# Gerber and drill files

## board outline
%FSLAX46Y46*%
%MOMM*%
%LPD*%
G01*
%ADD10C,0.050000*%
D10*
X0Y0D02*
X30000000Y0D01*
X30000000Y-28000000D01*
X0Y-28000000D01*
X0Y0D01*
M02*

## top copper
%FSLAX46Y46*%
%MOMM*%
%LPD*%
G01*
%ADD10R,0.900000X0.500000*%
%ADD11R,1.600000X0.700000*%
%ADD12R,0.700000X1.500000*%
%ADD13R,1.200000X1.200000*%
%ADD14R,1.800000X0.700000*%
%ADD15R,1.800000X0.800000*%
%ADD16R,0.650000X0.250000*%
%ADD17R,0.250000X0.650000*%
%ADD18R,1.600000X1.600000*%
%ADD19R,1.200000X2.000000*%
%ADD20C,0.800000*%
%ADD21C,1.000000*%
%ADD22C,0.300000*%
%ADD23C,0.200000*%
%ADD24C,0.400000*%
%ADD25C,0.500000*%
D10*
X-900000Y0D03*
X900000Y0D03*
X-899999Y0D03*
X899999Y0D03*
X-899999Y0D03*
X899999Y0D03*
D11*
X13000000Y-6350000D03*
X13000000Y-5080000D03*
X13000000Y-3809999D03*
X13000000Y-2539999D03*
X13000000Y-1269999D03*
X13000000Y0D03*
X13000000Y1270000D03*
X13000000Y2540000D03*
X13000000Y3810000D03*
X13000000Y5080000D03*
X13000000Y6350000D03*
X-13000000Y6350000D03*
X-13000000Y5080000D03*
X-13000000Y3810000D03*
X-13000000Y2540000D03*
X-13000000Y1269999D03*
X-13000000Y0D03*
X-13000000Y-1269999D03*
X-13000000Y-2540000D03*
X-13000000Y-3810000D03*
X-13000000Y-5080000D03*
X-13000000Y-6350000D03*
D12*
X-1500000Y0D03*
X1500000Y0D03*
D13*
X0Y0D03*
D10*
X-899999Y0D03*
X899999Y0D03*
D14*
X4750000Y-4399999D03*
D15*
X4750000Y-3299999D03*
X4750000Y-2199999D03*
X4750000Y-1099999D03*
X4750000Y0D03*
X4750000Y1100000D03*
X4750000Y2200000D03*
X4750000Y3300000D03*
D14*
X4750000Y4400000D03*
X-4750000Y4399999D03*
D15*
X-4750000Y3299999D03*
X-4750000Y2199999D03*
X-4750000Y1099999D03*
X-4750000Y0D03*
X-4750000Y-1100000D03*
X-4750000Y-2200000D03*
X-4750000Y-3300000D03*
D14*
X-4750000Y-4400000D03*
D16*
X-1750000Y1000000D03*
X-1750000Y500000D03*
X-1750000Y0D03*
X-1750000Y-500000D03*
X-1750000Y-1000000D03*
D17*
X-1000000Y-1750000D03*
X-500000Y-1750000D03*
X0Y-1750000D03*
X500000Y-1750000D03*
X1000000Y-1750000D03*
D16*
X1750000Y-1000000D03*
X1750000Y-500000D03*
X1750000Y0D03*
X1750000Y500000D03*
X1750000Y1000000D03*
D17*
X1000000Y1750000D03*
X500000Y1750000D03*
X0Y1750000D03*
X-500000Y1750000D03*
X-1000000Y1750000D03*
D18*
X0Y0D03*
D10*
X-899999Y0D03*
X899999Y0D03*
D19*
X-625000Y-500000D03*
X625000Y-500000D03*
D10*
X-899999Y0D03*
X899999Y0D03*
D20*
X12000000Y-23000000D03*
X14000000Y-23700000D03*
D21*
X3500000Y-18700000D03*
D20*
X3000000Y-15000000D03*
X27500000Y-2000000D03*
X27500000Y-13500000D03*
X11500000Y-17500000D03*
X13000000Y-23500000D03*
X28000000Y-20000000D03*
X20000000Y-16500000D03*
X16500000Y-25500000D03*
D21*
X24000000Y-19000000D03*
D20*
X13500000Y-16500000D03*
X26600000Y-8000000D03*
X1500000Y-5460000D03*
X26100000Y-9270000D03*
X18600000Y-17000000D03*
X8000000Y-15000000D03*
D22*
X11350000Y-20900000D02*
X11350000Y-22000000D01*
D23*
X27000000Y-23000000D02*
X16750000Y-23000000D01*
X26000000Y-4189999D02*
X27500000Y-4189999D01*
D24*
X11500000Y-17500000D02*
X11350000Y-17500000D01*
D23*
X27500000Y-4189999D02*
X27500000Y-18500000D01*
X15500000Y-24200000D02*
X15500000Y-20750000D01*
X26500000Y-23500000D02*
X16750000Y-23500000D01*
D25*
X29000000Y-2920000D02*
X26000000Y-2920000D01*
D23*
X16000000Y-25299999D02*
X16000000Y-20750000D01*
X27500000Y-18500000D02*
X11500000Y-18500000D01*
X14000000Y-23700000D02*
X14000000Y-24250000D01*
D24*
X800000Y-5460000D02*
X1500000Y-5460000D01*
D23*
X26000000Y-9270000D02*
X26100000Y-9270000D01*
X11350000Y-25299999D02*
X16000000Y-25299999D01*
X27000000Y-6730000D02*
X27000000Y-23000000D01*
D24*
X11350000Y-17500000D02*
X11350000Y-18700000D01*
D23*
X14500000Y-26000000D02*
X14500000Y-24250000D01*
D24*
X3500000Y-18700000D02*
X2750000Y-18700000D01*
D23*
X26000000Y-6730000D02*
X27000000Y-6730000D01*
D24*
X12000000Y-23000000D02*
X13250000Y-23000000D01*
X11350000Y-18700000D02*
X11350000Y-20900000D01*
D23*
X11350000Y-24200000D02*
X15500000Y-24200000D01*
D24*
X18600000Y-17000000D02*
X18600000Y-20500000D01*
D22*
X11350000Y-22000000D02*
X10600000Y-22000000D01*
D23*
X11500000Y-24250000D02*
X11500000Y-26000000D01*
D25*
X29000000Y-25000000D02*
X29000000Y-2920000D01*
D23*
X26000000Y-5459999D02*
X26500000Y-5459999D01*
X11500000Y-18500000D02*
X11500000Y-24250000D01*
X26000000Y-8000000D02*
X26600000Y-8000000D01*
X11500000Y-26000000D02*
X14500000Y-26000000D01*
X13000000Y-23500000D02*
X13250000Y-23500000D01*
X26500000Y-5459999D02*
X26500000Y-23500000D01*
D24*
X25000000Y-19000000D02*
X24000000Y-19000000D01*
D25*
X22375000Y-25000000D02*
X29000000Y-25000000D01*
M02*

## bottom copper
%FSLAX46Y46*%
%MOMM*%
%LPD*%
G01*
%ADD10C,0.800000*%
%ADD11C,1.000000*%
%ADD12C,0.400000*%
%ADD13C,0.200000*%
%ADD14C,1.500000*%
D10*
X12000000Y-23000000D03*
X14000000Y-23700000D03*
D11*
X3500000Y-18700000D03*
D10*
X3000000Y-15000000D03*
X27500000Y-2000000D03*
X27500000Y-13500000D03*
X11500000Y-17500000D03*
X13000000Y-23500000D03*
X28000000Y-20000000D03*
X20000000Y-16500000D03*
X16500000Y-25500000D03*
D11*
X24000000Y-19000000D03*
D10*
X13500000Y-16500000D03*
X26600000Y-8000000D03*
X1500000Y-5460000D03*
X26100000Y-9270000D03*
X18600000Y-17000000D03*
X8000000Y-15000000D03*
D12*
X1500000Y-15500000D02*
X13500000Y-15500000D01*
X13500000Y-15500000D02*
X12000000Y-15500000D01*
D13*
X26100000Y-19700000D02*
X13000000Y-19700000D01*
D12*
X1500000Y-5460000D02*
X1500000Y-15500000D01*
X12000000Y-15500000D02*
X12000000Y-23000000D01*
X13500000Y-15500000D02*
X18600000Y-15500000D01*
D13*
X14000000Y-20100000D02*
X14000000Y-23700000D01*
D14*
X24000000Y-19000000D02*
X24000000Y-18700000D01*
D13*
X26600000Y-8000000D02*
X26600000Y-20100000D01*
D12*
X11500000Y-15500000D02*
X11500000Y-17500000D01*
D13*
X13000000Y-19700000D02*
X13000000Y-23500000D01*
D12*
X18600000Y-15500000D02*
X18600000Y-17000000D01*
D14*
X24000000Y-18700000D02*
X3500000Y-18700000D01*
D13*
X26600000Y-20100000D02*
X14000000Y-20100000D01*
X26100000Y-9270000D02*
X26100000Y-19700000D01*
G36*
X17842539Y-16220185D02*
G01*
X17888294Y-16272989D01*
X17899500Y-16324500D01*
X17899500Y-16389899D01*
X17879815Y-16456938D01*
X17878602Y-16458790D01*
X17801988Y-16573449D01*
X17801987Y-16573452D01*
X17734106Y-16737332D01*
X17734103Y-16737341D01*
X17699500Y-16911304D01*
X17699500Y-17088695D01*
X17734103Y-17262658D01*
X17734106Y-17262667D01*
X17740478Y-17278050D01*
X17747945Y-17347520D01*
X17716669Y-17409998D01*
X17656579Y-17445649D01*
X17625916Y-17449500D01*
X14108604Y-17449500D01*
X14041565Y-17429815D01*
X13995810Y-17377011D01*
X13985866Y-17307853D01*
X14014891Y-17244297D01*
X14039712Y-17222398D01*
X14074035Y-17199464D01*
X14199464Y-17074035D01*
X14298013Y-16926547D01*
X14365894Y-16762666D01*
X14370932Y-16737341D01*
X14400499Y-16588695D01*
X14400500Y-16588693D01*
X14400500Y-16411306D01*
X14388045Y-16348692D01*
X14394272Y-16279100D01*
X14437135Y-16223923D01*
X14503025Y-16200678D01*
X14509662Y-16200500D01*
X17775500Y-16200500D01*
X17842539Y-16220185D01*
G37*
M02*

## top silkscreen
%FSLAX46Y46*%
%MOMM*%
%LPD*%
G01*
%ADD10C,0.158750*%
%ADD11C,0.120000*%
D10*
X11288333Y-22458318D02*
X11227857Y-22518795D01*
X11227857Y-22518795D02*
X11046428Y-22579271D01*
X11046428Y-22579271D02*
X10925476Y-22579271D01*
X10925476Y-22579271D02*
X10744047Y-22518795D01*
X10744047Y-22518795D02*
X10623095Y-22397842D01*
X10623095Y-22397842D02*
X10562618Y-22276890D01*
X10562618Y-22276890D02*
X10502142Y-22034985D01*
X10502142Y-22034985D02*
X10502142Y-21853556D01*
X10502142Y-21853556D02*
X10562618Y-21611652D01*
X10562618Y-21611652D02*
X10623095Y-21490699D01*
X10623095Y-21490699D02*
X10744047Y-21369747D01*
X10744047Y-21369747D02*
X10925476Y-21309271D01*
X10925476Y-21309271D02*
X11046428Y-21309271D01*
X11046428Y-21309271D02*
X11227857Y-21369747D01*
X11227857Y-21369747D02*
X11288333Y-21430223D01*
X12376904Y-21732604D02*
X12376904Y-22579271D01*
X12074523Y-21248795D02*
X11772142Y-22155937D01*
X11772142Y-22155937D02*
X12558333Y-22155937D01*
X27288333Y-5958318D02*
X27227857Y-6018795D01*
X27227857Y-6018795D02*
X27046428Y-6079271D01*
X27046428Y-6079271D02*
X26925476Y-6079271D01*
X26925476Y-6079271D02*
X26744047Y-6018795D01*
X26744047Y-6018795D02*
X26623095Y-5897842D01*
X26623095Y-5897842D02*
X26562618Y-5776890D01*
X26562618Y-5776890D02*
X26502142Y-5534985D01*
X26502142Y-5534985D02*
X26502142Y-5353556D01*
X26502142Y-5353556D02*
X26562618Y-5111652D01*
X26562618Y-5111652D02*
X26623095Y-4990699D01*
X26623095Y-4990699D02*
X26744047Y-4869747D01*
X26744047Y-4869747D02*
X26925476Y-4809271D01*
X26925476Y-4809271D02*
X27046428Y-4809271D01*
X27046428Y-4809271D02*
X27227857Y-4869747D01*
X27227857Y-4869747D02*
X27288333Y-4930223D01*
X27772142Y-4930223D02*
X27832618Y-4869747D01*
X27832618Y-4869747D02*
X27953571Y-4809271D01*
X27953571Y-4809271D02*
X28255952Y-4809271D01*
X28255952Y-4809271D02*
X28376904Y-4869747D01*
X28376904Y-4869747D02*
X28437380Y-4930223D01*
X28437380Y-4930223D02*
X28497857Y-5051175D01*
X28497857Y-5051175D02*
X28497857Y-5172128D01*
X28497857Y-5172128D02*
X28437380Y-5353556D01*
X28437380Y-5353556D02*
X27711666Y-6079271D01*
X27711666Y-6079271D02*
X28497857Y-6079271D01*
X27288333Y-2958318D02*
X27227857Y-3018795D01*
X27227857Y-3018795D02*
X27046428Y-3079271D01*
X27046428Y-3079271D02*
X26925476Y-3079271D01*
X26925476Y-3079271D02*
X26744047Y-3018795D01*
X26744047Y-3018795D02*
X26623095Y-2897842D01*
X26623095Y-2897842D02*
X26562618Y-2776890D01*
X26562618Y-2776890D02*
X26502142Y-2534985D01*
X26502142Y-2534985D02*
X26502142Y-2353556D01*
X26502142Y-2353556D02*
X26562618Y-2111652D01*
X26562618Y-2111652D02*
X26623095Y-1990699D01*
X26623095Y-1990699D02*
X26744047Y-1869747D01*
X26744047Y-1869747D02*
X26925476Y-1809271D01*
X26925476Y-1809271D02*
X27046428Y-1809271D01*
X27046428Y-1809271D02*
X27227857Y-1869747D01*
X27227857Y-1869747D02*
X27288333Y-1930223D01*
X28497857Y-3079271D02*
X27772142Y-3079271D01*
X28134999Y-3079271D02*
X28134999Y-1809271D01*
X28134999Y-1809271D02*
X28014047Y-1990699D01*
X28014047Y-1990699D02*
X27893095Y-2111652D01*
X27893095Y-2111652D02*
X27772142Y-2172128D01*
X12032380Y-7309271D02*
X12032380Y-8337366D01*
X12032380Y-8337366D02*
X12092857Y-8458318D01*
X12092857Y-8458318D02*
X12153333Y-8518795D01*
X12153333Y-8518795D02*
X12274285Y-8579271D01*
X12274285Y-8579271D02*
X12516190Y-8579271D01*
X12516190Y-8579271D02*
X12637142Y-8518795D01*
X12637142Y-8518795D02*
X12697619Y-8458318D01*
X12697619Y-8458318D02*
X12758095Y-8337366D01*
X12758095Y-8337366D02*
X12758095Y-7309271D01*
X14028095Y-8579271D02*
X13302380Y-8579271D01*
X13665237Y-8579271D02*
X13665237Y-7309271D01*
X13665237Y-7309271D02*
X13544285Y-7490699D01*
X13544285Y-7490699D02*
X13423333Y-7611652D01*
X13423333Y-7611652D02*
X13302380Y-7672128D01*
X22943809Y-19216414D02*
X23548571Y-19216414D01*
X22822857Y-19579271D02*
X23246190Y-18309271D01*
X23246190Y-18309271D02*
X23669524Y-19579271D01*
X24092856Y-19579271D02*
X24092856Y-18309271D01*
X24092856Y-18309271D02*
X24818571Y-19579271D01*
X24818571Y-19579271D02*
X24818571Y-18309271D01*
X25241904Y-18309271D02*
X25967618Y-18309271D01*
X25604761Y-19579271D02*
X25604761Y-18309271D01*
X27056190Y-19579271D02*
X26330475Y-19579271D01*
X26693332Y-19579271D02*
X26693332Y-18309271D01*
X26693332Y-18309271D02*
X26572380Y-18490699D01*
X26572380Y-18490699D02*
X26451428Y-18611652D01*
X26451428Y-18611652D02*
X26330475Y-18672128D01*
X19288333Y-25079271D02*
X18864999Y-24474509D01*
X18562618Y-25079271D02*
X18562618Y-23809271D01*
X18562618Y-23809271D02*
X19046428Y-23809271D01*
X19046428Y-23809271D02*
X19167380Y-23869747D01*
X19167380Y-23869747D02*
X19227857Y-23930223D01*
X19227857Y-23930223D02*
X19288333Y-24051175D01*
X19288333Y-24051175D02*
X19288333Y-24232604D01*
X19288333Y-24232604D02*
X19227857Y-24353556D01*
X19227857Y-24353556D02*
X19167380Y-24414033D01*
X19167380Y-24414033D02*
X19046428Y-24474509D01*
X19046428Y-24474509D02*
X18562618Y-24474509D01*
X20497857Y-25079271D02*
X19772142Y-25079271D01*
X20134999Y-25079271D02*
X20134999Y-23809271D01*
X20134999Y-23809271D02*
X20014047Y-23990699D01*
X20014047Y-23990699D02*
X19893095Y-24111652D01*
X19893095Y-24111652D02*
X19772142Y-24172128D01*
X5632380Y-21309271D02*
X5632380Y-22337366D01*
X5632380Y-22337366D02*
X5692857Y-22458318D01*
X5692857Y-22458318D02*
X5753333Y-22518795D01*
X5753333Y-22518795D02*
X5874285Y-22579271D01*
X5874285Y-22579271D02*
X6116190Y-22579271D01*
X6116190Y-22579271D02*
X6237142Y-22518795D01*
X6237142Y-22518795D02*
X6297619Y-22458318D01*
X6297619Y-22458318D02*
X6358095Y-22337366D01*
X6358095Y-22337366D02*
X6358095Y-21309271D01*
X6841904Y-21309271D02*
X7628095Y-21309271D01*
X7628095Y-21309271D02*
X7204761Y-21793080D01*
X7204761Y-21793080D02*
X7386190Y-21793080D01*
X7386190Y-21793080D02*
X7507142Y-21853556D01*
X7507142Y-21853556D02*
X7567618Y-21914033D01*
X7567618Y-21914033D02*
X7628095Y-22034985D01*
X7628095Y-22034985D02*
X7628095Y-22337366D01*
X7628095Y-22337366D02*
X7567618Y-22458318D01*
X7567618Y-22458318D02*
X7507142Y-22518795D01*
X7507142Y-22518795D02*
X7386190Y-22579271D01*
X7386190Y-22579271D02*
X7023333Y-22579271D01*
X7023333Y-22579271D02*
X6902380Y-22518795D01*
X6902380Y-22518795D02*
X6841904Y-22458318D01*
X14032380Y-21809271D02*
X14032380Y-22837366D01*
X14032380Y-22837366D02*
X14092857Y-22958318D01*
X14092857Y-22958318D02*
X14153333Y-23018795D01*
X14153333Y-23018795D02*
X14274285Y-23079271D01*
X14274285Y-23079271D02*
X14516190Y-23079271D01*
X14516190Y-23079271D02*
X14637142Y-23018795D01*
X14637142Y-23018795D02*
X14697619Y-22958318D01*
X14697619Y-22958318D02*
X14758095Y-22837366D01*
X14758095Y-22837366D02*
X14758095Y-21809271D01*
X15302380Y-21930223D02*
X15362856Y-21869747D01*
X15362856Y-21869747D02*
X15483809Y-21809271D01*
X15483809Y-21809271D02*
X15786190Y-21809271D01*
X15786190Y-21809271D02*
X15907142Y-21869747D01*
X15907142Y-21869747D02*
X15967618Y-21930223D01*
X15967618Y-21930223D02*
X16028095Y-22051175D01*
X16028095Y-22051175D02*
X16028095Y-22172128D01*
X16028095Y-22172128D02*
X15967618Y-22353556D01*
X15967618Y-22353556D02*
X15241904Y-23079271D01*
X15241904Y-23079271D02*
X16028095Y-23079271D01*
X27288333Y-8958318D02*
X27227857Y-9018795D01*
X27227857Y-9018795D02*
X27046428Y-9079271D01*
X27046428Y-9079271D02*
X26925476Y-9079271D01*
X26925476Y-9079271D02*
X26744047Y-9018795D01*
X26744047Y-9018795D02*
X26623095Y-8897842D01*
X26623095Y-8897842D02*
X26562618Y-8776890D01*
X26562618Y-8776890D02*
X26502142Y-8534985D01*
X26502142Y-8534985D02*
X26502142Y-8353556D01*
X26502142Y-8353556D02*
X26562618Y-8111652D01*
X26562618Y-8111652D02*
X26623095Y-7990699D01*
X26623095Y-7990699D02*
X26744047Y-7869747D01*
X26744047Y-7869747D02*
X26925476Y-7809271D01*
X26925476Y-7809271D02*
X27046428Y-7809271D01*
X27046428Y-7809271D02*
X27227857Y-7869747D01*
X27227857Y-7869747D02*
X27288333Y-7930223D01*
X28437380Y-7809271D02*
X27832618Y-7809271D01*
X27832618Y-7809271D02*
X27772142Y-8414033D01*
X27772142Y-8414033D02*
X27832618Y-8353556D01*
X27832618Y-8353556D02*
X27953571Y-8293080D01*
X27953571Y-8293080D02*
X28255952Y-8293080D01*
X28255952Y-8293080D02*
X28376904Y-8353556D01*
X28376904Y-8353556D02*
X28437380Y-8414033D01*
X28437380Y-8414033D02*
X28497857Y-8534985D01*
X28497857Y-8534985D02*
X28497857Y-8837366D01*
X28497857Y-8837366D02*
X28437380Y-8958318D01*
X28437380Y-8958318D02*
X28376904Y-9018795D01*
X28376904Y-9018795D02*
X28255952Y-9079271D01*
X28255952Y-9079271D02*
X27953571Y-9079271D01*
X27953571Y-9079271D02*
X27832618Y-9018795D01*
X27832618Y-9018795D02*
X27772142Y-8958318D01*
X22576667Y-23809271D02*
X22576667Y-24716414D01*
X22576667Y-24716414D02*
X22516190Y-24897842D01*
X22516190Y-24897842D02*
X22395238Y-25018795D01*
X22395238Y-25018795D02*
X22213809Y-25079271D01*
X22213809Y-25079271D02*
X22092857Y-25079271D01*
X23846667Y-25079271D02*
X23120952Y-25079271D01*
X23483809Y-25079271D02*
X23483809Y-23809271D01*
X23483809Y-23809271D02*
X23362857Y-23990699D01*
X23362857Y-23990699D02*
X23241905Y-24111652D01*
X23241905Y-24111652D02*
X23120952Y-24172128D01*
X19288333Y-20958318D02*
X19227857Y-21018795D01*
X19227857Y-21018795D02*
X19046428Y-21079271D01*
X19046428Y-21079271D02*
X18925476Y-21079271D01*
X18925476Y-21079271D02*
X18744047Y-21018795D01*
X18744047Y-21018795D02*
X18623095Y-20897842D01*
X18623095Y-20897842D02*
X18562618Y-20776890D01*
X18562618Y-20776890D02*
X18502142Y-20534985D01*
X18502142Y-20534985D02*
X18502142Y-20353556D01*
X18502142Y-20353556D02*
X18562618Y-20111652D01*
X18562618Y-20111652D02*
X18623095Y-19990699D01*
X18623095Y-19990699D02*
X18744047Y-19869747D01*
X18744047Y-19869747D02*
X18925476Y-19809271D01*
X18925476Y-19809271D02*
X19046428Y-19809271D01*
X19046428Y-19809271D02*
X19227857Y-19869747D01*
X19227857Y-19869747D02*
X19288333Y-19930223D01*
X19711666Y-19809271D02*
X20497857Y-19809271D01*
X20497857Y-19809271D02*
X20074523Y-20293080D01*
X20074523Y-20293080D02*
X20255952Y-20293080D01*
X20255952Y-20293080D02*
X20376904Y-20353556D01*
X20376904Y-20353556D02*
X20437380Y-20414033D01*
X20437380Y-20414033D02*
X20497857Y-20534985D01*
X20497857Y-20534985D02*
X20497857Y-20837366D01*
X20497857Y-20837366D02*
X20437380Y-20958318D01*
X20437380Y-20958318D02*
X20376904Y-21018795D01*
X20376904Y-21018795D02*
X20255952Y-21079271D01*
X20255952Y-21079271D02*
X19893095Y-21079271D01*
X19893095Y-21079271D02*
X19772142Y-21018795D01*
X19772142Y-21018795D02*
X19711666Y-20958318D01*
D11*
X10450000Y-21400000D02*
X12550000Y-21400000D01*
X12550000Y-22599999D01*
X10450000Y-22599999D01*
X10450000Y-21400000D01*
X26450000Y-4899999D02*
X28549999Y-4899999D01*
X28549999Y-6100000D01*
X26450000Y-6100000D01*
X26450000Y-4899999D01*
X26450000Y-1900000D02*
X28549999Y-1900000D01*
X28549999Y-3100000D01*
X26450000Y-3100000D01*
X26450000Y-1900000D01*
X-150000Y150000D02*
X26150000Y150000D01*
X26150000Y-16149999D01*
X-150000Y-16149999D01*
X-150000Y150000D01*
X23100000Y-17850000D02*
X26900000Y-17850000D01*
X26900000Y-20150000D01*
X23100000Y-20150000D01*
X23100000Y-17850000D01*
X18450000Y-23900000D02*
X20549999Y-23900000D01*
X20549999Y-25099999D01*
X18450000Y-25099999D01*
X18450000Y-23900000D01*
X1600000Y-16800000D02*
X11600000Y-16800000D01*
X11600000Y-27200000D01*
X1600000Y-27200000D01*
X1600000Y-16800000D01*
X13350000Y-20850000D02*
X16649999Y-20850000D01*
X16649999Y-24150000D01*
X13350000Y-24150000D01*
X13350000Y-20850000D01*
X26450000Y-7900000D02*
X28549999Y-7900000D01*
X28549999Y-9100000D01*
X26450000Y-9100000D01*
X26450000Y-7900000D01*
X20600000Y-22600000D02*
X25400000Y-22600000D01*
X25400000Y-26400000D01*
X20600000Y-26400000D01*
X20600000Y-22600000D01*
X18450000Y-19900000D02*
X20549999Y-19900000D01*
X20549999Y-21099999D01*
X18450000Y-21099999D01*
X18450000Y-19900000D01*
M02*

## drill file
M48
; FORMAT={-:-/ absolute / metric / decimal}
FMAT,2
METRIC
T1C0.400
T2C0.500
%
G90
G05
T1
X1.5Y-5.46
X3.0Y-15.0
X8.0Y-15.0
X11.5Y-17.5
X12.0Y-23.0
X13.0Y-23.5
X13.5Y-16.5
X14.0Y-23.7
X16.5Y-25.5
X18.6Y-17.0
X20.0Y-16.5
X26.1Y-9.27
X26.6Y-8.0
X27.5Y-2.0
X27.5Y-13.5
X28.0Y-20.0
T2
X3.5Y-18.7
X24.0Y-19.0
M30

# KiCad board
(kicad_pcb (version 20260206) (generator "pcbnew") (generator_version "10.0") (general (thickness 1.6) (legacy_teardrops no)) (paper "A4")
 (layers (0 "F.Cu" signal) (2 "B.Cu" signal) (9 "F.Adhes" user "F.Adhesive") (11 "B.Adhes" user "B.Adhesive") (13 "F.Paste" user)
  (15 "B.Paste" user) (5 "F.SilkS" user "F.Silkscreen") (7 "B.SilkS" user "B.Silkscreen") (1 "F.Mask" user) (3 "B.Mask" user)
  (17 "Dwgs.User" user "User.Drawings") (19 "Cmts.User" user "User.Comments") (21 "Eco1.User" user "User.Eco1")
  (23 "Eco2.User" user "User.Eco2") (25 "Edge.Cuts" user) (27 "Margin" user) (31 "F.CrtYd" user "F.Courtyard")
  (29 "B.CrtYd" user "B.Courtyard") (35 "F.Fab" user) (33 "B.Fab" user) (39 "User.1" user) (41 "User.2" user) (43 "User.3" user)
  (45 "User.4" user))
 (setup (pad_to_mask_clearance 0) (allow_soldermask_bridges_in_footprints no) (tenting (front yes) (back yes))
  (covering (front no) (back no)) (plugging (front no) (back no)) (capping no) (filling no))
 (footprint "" (layer "F.Cu") (at 11.5 22)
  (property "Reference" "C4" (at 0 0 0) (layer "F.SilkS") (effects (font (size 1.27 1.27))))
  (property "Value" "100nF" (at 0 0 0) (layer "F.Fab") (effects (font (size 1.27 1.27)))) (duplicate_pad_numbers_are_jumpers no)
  (fp_rect (start -1.05 -0.6) (end 1.05 0.599999) (stroke (width 0.12) (type default)) (fill no) (layer "F.SilkS"))
  (pad "1" smd rect (at -12.4 -22) (size 0.9 0.5) (layers "F.Cu" "F.Mask" "F.Paste") (thermal_bridge_angle 45))
  (pad "2" smd rect (at -10.6 -22) (size 0.9 0.5) (layers "F.Cu" "F.Mask" "F.Paste") (thermal_bridge_angle 45)))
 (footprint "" (layer "F.Cu") (at 27.5 5.5)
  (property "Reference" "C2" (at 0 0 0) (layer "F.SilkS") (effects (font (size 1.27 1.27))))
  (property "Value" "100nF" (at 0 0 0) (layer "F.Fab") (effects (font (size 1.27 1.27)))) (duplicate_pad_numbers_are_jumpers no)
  (fp_rect (start -1.05 -0.600001) (end 1.049999 0.6) (stroke (width 0.12) (type default)) (fill no) (layer "F.SilkS"))
  (pad "1" smd rect (at -28.399999 -5.5) (size 0.9 0.5) (layers "F.Cu" "F.Mask" "F.Paste") (thermal_bridge_angle 45))
  (pad "2" smd rect (at -26.600001 -5.5) (size 0.9 0.5) (layers "F.Cu" "F.Mask" "F.Paste") (thermal_bridge_angle 45)))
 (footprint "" (layer "F.Cu") (at 27.5 2.5)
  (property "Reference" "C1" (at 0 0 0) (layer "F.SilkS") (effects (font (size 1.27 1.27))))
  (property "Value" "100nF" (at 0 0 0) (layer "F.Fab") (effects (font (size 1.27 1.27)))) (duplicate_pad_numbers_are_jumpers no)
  (fp_rect (start -1.05 -0.6) (end 1.049999 0.6) (stroke (width 0.12) (type default)) (fill no) (layer "F.SilkS"))
  (pad "1" smd rect (at -28.399999 -2.5) (size 0.9 0.5) (layers "F.Cu" "F.Mask" "F.Paste") (thermal_bridge_angle 45))
  (pad "2" smd rect (at -26.600001 -2.5) (size 0.9 0.5) (layers "F.Cu" "F.Mask" "F.Paste") (thermal_bridge_angle 45)))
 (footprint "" (layer "F.Cu") (at 13 8)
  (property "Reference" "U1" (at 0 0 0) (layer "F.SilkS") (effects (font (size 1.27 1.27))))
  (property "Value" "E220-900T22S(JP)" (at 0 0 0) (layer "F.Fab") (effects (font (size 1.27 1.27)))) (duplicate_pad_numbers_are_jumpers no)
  (fp_rect (start -13.15 -8.15) (end 13.15 8.149999) (stroke (width 0.12) (type default)) (fill no) (layer "F.SilkS"))
  (pad "1" smd rect (at 0 -1.65) (size 1.6 0.7) (layers "F.Cu" "F.Mask" "F.Paste") (thermal_bridge_angle 45))
  (pad "2" smd rect (at 0 -2.92) (size 1.6 0.7) (layers "F.Cu" "F.Mask" "F.Paste") (thermal_bridge_angle 45))
  (pad "3" smd rect (at 0 -4.190001) (size 1.6 0.7) (layers "F.Cu" "F.Mask" "F.Paste") (thermal_bridge_angle 45))
  (pad "4" smd rect (at 0 -5.460001) (size 1.6 0.7) (layers "F.Cu" "F.Mask" "F.Paste") (thermal_bridge_angle 45))
  (pad "5" smd rect (at 0 -6.730001) (size 1.6 0.7) (layers "F.Cu" "F.Mask" "F.Paste") (thermal_bridge_angle 45))
  (pad "6" smd rect (at 0 -8) (size 1.6 0.7) (layers "F.Cu" "F.Mask" "F.Paste") (thermal_bridge_angle 45))
  (pad "7" smd rect (at 0 -9.27) (size 1.6 0.7) (layers "F.Cu" "F.Mask" "F.Paste") (thermal_bridge_angle 45))
  (pad "8" smd rect (at 0 -10.54) (size 1.6 0.7) (layers "F.Cu" "F.Mask" "F.Paste") (thermal_bridge_angle 45))
  (pad "9" smd rect (at 0 -11.81) (size 1.6 0.7) (layers "F.Cu" "F.Mask" "F.Paste") (thermal_bridge_angle 45))
  (pad "10" smd rect (at 0 -13.08) (size 1.6 0.7) (layers "F.Cu" "F.Mask" "F.Paste") (thermal_bridge_angle 45))
  (pad "11" smd rect (at 0 -14.35) (size 1.6 0.7) (layers "F.Cu" "F.Mask" "F.Paste") (thermal_bridge_angle 45))
  (pad "12" smd rect (at -26 -14.35) (size 1.6 0.7) (layers "F.Cu" "F.Mask" "F.Paste") (thermal_bridge_angle 45))
  (pad "13" smd rect (at -26 -13.08) (size 1.6 0.7) (layers "F.Cu" "F.Mask" "F.Paste") (thermal_bridge_angle 45))
  (pad "14" smd rect (at -26 -11.81) (size 1.6 0.7) (layers "F.Cu" "F.Mask" "F.Paste") (thermal_bridge_angle 45))
  (pad "15" smd rect (at -26 -10.54) (size 1.6 0.7) (layers "F.Cu" "F.Mask" "F.Paste") (thermal_bridge_angle 45))
  (pad "16" smd rect (at -26 -9.269999) (size 1.6 0.7) (layers "F.Cu" "F.Mask" "F.Paste") (thermal_bridge_angle 45))
  (pad "17" smd rect (at -26 -8) (size 1.6 0.7) (layers "F.Cu" "F.Mask" "F.Paste") (thermal_bridge_angle 45))
  (pad "18" smd rect (at -26 -6.730001) (size 1.6 0.7) (layers "F.Cu" "F.Mask" "F.Paste") (thermal_bridge_angle 45))
  (pad "19" smd rect (at -26 -5.46) (size 1.6 0.7) (layers "F.Cu" "F.Mask" "F.Paste") (thermal_bridge_angle 45))
  (pad "20" smd rect (at -26 -4.19) (size 1.6 0.7) (layers "F.Cu" "F.Mask" "F.Paste") (thermal_bridge_angle 45))
  (pad "21" smd rect (at -26 -2.92) (size 1.6 0.7) (layers "F.Cu" "F.Mask" "F.Paste") (thermal_bridge_angle 45))
  (pad "22" smd rect (at -26 -1.65) (size 1.6 0.7) (layers "F.Cu" "F.Mask" "F.Paste") (thermal_bridge_angle 45)))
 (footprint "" (layer "F.Cu") (at 25 19)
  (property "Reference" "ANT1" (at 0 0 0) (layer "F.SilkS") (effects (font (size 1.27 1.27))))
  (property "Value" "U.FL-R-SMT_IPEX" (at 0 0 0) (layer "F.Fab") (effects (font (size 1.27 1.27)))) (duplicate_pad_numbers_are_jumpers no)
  (fp_rect (start -1.9 -1.15) (end 1.9 1.15) (stroke (width 0.12) (type default)) (fill no) (layer "F.SilkS"))
  (pad "G1" smd rect (at -26.5 -19) (size 0.7 1.5) (layers "F.Cu" "F.Mask" "F.Paste") (thermal_bridge_angle 45))
  (pad "G2" smd rect (at -23.5 -19) (size 0.7 1.5) (layers "F.Cu" "F.Mask" "F.Paste") (thermal_bridge_angle 45))
  (pad "S" smd rect (at -25 -19) (size 1.2 1.2) (layers "F.Cu" "F.Mask" "F.Paste") (thermal_bridge_angle 45)))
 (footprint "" (layer "F.Cu") (at 19.5 24.5)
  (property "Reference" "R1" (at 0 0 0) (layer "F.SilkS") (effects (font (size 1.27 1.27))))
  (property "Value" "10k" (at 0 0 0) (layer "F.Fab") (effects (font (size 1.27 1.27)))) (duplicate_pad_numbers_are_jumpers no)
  (fp_rect (start -1.05 -0.6) (end 1.049999 0.599999) (stroke (width 0.12) (type default)) (fill no) (layer "F.SilkS"))
  (pad "1" smd rect (at -20.399999 -24.5) (size 0.9 0.5) (layers "F.Cu" "F.Mask" "F.Paste") (thermal_bridge_angle 45))
  (pad "2" smd rect (at -18.600001 -24.5) (size 0.9 0.5) (layers "F.Cu" "F.Mask" "F.Paste") (thermal_bridge_angle 45)))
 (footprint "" (layer "F.Cu") (at 6.6 22)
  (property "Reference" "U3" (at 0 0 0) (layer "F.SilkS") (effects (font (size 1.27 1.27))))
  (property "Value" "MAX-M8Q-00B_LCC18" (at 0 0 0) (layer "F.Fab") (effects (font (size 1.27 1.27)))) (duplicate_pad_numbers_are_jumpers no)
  (fp_rect (start -5 -5.2) (end 5 5.2) (stroke (width 0.12) (type default)) (fill no) (layer "F.SilkS"))
  (pad "1" smd rect (at -1.85 -17.600001) (size 1.8 0.7) (layers "F.Cu" "F.Mask" "F.Paste") (thermal_bridge_angle 45))
  (pad "2" smd rect (at -1.85 -18.700001) (size 1.8 0.8) (layers "F.Cu" "F.Mask" "F.Paste") (thermal_bridge_angle 45))
  (pad "3" smd rect (at -1.85 -19.800001) (size 1.8 0.8) (layers "F.Cu" "F.Mask" "F.Paste") (thermal_bridge_angle 45))
  (pad "4" smd rect (at -1.85 -20.900001) (size 1.8 0.8) (layers "F.Cu" "F.Mask" "F.Paste") (thermal_bridge_angle 45))
  (pad "5" smd rect (at -1.85 -22) (size 1.8 0.8) (layers "F.Cu" "F.Mask" "F.Paste") (thermal_bridge_angle 45))
  (pad "6" smd rect (at -1.85 -23.1) (size 1.8 0.8) (layers "F.Cu" "F.Mask" "F.Paste") (thermal_bridge_angle 45))
  (pad "7" smd rect (at -1.85 -24.2) (size 1.8 0.8) (layers "F.Cu" "F.Mask" "F.Paste") (thermal_bridge_angle 45))
  (pad "8" smd rect (at -1.85 -25.3) (size 1.8 0.8) (layers "F.Cu" "F.Mask" "F.Paste") (thermal_bridge_angle 45))
  (pad "9" smd rect (at -1.85 -26.4) (size 1.8 0.7) (layers "F.Cu" "F.Mask" "F.Paste") (thermal_bridge_angle 45))
  (pad "10" smd rect (at -11.35 -26.399999) (size 1.8 0.7) (layers "F.Cu" "F.Mask" "F.Paste") (thermal_bridge_angle 45))
  (pad "11" smd rect (at -11.35 -25.299999) (size 1.8 0.8) (layers "F.Cu" "F.Mask" "F.Paste") (thermal_bridge_angle 45))
  (pad "12" smd rect (at -11.35 -24.199999) (size 1.8 0.8) (layers "F.Cu" "F.Mask" "F.Paste") (thermal_bridge_angle 45))
  (pad "13" smd rect (at -11.35 -23.099999) (size 1.8 0.8) (layers "F.Cu" "F.Mask" "F.Paste") (thermal_bridge_angle 45))
  (pad "14" smd rect (at -11.35 -22) (size 1.8 0.8) (layers "F.Cu" "F.Mask" "F.Paste") (thermal_bridge_angle 45))
  (pad "15" smd rect (at -11.35 -20.9) (size 1.8 0.8) (layers "F.Cu" "F.Mask" "F.Paste") (thermal_bridge_angle 45))
  (pad "16" smd rect (at -11.35 -19.8) (size 1.8 0.8) (layers "F.Cu" "F.Mask" "F.Paste") (thermal_bridge_angle 45))
  (pad "17" smd rect (at -11.35 -18.7) (size 1.8 0.8) (layers "F.Cu" "F.Mask" "F.Paste") (thermal_bridge_angle 45))
  (pad "18" smd rect (at -11.35 -17.6) (size 1.8 0.7) (layers "F.Cu" "F.Mask" "F.Paste") (thermal_bridge_angle 45)))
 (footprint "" (layer "F.Cu") (at 15 22.5)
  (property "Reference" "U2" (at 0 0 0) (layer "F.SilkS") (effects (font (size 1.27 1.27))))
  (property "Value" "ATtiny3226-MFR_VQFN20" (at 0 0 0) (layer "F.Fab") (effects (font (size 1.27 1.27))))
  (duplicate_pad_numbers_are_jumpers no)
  (fp_rect (start -1.65 -1.65) (end 1.649999 1.65) (stroke (width 0.12) (type default)) (fill no) (layer "F.SilkS"))
  (pad "1" smd rect (at -16.75 -23.5) (size 0.65 0.25) (layers "F.Cu" "F.Mask" "F.Paste") (thermal_bridge_angle 45))
  (pad "2" smd rect (at -16.75 -23) (size 0.65 0.25) (layers "F.Cu" "F.Mask" "F.Paste") (thermal_bridge_angle 45))
  (pad "3" smd rect (at -16.75 -22.5) (size 0.65 0.25) (layers "F.Cu" "F.Mask" "F.Paste") (thermal_bridge_angle 45))
  (pad "4" smd rect (at -16.75 -22) (size 0.65 0.25) (layers "F.Cu" "F.Mask" "F.Paste") (thermal_bridge_angle 45))
  (pad "5" smd rect (at -16.75 -21.5) (size 0.65 0.25) (layers "F.Cu" "F.Mask" "F.Paste") (thermal_bridge_angle 45))
  (pad "6" smd rect (at -16 -20.75) (size 0.25 0.65) (layers "F.Cu" "F.Mask" "F.Paste") (thermal_bridge_angle 45))
  (pad "7" smd rect (at -15.5 -20.75) (size 0.25 0.65) (layers "F.Cu" "F.Mask" "F.Paste") (thermal_bridge_angle 45))
  (pad "8" smd rect (at -15 -20.75) (size 0.25 0.65) (layers "F.Cu" "F.Mask" "F.Paste") (thermal_bridge_angle 45))
  (pad "9" smd rect (at -14.5 -20.75) (size 0.25 0.65) (layers "F.Cu" "F.Mask" "F.Paste") (thermal_bridge_angle 45))
  (pad "10" smd rect (at -14 -20.75) (size 0.25 0.65) (layers "F.Cu" "F.Mask" "F.Paste") (thermal_bridge_angle 45))
  (pad "11" smd rect (at -13.25 -21.5) (size 0.65 0.25) (layers "F.Cu" "F.Mask" "F.Paste") (thermal_bridge_angle 45))
  (pad "12" smd rect (at -13.25 -22) (size 0.65 0.25) (layers "F.Cu" "F.Mask" "F.Paste") (thermal_bridge_angle 45))
  (pad "13" smd rect (at -13.25 -22.5) (size 0.65 0.25) (layers "F.Cu" "F.Mask" "F.Paste") (thermal_bridge_angle 45))
  (pad "14" smd rect (at -13.25 -23) (size 0.65 0.25) (layers "F.Cu" "F.Mask" "F.Paste") (thermal_bridge_angle 45))
  (pad "15" smd rect (at -13.25 -23.5) (size 0.65 0.25) (layers "F.Cu" "F.Mask" "F.Paste") (thermal_bridge_angle 45))
  (pad "16" smd rect (at -14 -24.25) (size 0.25 0.65) (layers "F.Cu" "F.Mask" "F.Paste") (thermal_bridge_angle 45))
  (pad "17" smd rect (at -14.5 -24.25) (size 0.25 0.65) (layers "F.Cu" "F.Mask" "F.Paste") (thermal_bridge_angle 45))
  (pad "18" smd rect (at -15 -24.25) (size 0.25 0.65) (layers "F.Cu" "F.Mask" "F.Paste") (thermal_bridge_angle 45))
  (pad "19" smd rect (at -15.5 -24.25) (size 0.25 0.65) (layers "F.Cu" "F.Mask" "F.Paste") (thermal_bridge_angle 45))
  (pad "20" smd rect (at -16 -24.25) (size 0.25 0.65) (layers "F.Cu" "F.Mask" "F.Paste") (thermal_bridge_angle 45))
  (pad "EP" smd rect (at -15 -22.5) (size 1.6 1.6) (layers "F.Cu" "F.Mask" "F.Paste") (thermal_bridge_angle 45)))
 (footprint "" (layer "F.Cu") (at 27.5 8.5)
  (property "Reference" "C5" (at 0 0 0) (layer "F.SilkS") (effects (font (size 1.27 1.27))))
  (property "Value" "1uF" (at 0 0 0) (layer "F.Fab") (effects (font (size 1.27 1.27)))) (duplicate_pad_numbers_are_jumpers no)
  (fp_rect (start -1.05 -0.6) (end 1.049999 0.6) (stroke (width 0.12) (type default)) (fill no) (layer "F.SilkS"))
  (pad "1" smd rect (at -28.399999 -8.5) (size 0.9 0.5) (layers "F.Cu" "F.Mask" "F.Paste") (thermal_bridge_angle 45))
  (pad "2" smd rect (at -26.600001 -8.5) (size 0.9 0.5) (layers "F.Cu" "F.Mask" "F.Paste") (thermal_bridge_angle 45)))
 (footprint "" (layer "F.Cu") (at 23 24.5)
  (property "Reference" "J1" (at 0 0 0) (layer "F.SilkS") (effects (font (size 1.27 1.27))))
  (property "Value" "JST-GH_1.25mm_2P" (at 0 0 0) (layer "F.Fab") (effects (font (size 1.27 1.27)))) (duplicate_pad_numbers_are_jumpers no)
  (fp_rect (start -2.4 -1.9) (end 2.4 1.9) (stroke (width 0.12) (type default)) (fill no) (layer "F.SilkS"))
  (pad "1" smd rect (at -23.625 -24) (size 1.2 2) (layers "F.Cu" "F.Mask" "F.Paste") (thermal_bridge_angle 45))
  (pad "2" smd rect (at -22.375 -24) (size 1.2 2) (layers "F.Cu" "F.Mask" "F.Paste") (thermal_bridge_angle 45)))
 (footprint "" (layer "F.Cu") (at 19.5 20.5)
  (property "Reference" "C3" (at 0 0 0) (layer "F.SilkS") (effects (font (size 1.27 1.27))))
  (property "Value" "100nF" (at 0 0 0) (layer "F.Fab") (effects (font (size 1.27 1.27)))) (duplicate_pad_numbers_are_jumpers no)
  (fp_rect (start -1.05 -0.6) (end 1.049999 0.599999) (stroke (width 0.12) (type default)) (fill no) (layer "F.SilkS"))
  (pad "1" smd rect (at -20.399999 -20.5) (size 0.9 0.5) (layers "F.Cu" "F.Mask" "F.Paste") (thermal_bridge_angle 45))
  (pad "2" smd rect (at -18.600001 -20.5) (size 0.9 0.5) (layers "F.Cu" "F.Mask" "F.Paste") (thermal_bridge_angle 45)))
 (gr_rect (start 0 0) (end 30 28) (stroke (width 0.05) (type default)) (fill no) (layer "Edge.Cuts"))
 (segment (start 11.35 20.9) (end 11.35 22) (width 0.3) (layer "F.Cu") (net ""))
 (segment (start 27 23) (end 16.75 23) (width 0.2) (layer "F.Cu") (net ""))
 (segment (start 26 4.189999) (end 27.5 4.189999) (width 0.2) (layer "F.Cu") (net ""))
 (segment (start 11.5 17.5) (end 11.35 17.5) (width 0.4) (layer "F.Cu") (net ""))
 (segment (start 27.5 4.189999) (end 27.5 18.5) (width 0.2) (layer "F.Cu") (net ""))
 (segment (start 15.5 24.2) (end 15.5 20.75) (width 0.2) (layer "F.Cu") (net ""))
 (segment (start 26.5 23.5) (end 16.75 23.5) (width 0.2) (layer "F.Cu") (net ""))
 (segment (start 29 2.92) (end 26 2.92) (width 0.5) (layer "F.Cu") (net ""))
 (segment (start 16 25.299999) (end 16 20.75) (width 0.2) (layer "F.Cu") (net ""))
 (segment (start 27.5 18.5) (end 11.5 18.5) (width 0.2) (layer "F.Cu") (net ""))
 (segment (start 14 23.7) (end 14 24.25) (width 0.2) (layer "F.Cu") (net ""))
 (segment (start 0.8 5.46) (end 1.5 5.46) (width 0.4) (layer "F.Cu") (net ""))
 (segment (start 26 9.27) (end 26.1 9.27) (width 0.2) (layer "F.Cu") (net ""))
 (segment (start 11.35 25.299999) (end 16 25.299999) (width 0.2) (layer "F.Cu") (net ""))
 (segment (start 27 6.73) (end 27 23) (width 0.2) (layer "F.Cu") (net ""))
 (segment (start 11.35 17.5) (end 11.35 18.7) (width 0.4) (layer "F.Cu") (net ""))
 (segment (start 14.5 26) (end 14.5 24.25) (width 0.2) (layer "F.Cu") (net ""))
 (segment (start 3.5 18.7) (end 2.75 18.7) (width 0.4) (layer "F.Cu") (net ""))
 (segment (start 26 6.73) (end 27 6.73) (width 0.2) (layer "F.Cu") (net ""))
 (segment (start 12 23) (end 13.25 23) (width 0.4) (layer "F.Cu") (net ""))
 (segment (start 11.35 18.7) (end 11.35 20.9) (width 0.4) (layer "F.Cu") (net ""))
 (segment (start 11.35 24.2) (end 15.5 24.2) (width 0.2) (layer "F.Cu") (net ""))
 (segment (start 18.6 17) (end 18.6 20.5) (width 0.4) (layer "F.Cu") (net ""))
 (segment (start 11.35 22) (end 10.6 22) (width 0.3) (layer "F.Cu") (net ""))
 (segment (start 11.5 24.25) (end 11.5 26) (width 0.2) (layer "F.Cu") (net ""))
 (segment (start 29 25) (end 29 2.92) (width 0.5) (layer "F.Cu") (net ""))
 (segment (start 26 5.459999) (end 26.5 5.459999) (width 0.2) (layer "F.Cu") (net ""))
 (segment (start 11.5 18.5) (end 11.5 24.25) (width 0.2) (layer "F.Cu") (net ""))
 (segment (start 26 8) (end 26.6 8) (width 0.2) (layer "F.Cu") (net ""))
 (segment (start 11.5 26) (end 14.5 26) (width 0.2) (layer "F.Cu") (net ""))
 (segment (start 13 23.5) (end 13.25 23.5) (width 0.2) (layer "F.Cu") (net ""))
 (segment (start 26.5 5.459999) (end 26.5 23.5) (width 0.2) (layer "F.Cu") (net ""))
 (segment (start 25 19) (end 24 19) (width 0.4) (layer "F.Cu") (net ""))
 (segment (start 22.375 25) (end 29 25) (width 0.5) (layer "F.Cu") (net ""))
 (via (at 12 23) (size 0.8) (drill 0.4) (layers "F.Cu" "B.Cu") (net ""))
 (via (at 14 23.7) (size 0.8) (drill 0.4) (layers "F.Cu" "B.Cu") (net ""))
 (via (at 3.5 18.7) (size 1) (drill 0.5) (layers "F.Cu" "B.Cu") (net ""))
 (via (at 3 15) (size 0.8) (drill 0.4) (layers "F.Cu" "B.Cu") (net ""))
 (via (at 27.5 2) (size 0.8) (drill 0.4) (layers "F.Cu" "B.Cu") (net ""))
 (via (at 27.5 13.5) (size 0.8) (drill 0.4) (layers "F.Cu" "B.Cu") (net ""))
 (via (at 11.5 17.5) (size 0.8) (drill 0.4) (layers "F.Cu" "B.Cu") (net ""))
 (via (at 13 23.5) (size 0.8) (drill 0.4) (layers "F.Cu" "B.Cu") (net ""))
 (via (at 28 20) (size 0.8) (drill 0.4) (layers "F.Cu" "B.Cu") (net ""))
 (via (at 20 16.5) (size 0.8) (drill 0.4) (layers "F.Cu" "B.Cu") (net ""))
 (via (at 16.5 25.5) (size 0.8) (drill 0.4) (layers "F.Cu" "B.Cu") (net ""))
 (via (at 24 19) (size 1) (drill 0.5) (layers "F.Cu" "B.Cu") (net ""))
 (via (at 13.5 16.5) (size 0.8) (drill 0.4) (layers "F.Cu" "B.Cu") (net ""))
 (via (at 26.6 8) (size 0.8) (drill 0.4) (layers "F.Cu" "B.Cu") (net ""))
 (via (at 1.5 5.46) (size 0.8) (drill 0.4) (layers "F.Cu" "B.Cu") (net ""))
 (via (at 26.1 9.27) (size 0.8) (drill 0.4) (layers "F.Cu" "B.Cu") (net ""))
 (via (at 18.6 17) (size 0.8) (drill 0.4) (layers "F.Cu" "B.Cu") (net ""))
 (via (at 8 15) (size 0.8) (drill 0.4) (layers "F.Cu" "B.Cu") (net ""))
 (segment (start 1.5 15.5) (end 13.5 15.5) (width 0.4) (layer "B.Cu") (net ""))
 (segment (start 13.5 15.5) (end 12 15.5) (width 0.4) (layer "B.Cu") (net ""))
 (segment (start 26.1 19.7) (end 13 19.7) (width 0.2) (layer "B.Cu") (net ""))
 (segment (start 1.5 5.46) (end 1.5 15.5) (width 0.4) (layer "B.Cu") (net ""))
 (segment (start 12 15.5) (end 12 23) (width 0.4) (layer "B.Cu") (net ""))
 (segment (start 13.5 15.5) (end 18.6 15.5) (width 0.4) (layer "B.Cu") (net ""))
 (segment (start 14 20.1) (end 14 23.7) (width 0.2) (layer "B.Cu") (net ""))
 (segment (start 24 19) (end 24 18.7) (width 1.5) (layer "B.Cu") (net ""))
 (segment (start 26.6 8) (end 26.6 20.1) (width 0.2) (layer "B.Cu") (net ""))
 (segment (start 11.5 15.5) (end 11.5 17.5) (width 0.4) (layer "B.Cu") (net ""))
 (segment (start 13 19.7) (end 13 23.5) (width 0.2) (layer "B.Cu") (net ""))
 (segment (start 18.6 15.5) (end 18.6 17) (width 0.4) (layer "B.Cu") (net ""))
 (segment (start 24 18.7) (end 3.5 18.7) (width 1.5) (layer "B.Cu") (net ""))
 (segment (start 26.6 20.1) (end 14 20.1) (width 0.2) (layer "B.Cu") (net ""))
 (segment (start 26.1 9.27) (end 26.1 19.7) (width 0.2) (layer "B.Cu") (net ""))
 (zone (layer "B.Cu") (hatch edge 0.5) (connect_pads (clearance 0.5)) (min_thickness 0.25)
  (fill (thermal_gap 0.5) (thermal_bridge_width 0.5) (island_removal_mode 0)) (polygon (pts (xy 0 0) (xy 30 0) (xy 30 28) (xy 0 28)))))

